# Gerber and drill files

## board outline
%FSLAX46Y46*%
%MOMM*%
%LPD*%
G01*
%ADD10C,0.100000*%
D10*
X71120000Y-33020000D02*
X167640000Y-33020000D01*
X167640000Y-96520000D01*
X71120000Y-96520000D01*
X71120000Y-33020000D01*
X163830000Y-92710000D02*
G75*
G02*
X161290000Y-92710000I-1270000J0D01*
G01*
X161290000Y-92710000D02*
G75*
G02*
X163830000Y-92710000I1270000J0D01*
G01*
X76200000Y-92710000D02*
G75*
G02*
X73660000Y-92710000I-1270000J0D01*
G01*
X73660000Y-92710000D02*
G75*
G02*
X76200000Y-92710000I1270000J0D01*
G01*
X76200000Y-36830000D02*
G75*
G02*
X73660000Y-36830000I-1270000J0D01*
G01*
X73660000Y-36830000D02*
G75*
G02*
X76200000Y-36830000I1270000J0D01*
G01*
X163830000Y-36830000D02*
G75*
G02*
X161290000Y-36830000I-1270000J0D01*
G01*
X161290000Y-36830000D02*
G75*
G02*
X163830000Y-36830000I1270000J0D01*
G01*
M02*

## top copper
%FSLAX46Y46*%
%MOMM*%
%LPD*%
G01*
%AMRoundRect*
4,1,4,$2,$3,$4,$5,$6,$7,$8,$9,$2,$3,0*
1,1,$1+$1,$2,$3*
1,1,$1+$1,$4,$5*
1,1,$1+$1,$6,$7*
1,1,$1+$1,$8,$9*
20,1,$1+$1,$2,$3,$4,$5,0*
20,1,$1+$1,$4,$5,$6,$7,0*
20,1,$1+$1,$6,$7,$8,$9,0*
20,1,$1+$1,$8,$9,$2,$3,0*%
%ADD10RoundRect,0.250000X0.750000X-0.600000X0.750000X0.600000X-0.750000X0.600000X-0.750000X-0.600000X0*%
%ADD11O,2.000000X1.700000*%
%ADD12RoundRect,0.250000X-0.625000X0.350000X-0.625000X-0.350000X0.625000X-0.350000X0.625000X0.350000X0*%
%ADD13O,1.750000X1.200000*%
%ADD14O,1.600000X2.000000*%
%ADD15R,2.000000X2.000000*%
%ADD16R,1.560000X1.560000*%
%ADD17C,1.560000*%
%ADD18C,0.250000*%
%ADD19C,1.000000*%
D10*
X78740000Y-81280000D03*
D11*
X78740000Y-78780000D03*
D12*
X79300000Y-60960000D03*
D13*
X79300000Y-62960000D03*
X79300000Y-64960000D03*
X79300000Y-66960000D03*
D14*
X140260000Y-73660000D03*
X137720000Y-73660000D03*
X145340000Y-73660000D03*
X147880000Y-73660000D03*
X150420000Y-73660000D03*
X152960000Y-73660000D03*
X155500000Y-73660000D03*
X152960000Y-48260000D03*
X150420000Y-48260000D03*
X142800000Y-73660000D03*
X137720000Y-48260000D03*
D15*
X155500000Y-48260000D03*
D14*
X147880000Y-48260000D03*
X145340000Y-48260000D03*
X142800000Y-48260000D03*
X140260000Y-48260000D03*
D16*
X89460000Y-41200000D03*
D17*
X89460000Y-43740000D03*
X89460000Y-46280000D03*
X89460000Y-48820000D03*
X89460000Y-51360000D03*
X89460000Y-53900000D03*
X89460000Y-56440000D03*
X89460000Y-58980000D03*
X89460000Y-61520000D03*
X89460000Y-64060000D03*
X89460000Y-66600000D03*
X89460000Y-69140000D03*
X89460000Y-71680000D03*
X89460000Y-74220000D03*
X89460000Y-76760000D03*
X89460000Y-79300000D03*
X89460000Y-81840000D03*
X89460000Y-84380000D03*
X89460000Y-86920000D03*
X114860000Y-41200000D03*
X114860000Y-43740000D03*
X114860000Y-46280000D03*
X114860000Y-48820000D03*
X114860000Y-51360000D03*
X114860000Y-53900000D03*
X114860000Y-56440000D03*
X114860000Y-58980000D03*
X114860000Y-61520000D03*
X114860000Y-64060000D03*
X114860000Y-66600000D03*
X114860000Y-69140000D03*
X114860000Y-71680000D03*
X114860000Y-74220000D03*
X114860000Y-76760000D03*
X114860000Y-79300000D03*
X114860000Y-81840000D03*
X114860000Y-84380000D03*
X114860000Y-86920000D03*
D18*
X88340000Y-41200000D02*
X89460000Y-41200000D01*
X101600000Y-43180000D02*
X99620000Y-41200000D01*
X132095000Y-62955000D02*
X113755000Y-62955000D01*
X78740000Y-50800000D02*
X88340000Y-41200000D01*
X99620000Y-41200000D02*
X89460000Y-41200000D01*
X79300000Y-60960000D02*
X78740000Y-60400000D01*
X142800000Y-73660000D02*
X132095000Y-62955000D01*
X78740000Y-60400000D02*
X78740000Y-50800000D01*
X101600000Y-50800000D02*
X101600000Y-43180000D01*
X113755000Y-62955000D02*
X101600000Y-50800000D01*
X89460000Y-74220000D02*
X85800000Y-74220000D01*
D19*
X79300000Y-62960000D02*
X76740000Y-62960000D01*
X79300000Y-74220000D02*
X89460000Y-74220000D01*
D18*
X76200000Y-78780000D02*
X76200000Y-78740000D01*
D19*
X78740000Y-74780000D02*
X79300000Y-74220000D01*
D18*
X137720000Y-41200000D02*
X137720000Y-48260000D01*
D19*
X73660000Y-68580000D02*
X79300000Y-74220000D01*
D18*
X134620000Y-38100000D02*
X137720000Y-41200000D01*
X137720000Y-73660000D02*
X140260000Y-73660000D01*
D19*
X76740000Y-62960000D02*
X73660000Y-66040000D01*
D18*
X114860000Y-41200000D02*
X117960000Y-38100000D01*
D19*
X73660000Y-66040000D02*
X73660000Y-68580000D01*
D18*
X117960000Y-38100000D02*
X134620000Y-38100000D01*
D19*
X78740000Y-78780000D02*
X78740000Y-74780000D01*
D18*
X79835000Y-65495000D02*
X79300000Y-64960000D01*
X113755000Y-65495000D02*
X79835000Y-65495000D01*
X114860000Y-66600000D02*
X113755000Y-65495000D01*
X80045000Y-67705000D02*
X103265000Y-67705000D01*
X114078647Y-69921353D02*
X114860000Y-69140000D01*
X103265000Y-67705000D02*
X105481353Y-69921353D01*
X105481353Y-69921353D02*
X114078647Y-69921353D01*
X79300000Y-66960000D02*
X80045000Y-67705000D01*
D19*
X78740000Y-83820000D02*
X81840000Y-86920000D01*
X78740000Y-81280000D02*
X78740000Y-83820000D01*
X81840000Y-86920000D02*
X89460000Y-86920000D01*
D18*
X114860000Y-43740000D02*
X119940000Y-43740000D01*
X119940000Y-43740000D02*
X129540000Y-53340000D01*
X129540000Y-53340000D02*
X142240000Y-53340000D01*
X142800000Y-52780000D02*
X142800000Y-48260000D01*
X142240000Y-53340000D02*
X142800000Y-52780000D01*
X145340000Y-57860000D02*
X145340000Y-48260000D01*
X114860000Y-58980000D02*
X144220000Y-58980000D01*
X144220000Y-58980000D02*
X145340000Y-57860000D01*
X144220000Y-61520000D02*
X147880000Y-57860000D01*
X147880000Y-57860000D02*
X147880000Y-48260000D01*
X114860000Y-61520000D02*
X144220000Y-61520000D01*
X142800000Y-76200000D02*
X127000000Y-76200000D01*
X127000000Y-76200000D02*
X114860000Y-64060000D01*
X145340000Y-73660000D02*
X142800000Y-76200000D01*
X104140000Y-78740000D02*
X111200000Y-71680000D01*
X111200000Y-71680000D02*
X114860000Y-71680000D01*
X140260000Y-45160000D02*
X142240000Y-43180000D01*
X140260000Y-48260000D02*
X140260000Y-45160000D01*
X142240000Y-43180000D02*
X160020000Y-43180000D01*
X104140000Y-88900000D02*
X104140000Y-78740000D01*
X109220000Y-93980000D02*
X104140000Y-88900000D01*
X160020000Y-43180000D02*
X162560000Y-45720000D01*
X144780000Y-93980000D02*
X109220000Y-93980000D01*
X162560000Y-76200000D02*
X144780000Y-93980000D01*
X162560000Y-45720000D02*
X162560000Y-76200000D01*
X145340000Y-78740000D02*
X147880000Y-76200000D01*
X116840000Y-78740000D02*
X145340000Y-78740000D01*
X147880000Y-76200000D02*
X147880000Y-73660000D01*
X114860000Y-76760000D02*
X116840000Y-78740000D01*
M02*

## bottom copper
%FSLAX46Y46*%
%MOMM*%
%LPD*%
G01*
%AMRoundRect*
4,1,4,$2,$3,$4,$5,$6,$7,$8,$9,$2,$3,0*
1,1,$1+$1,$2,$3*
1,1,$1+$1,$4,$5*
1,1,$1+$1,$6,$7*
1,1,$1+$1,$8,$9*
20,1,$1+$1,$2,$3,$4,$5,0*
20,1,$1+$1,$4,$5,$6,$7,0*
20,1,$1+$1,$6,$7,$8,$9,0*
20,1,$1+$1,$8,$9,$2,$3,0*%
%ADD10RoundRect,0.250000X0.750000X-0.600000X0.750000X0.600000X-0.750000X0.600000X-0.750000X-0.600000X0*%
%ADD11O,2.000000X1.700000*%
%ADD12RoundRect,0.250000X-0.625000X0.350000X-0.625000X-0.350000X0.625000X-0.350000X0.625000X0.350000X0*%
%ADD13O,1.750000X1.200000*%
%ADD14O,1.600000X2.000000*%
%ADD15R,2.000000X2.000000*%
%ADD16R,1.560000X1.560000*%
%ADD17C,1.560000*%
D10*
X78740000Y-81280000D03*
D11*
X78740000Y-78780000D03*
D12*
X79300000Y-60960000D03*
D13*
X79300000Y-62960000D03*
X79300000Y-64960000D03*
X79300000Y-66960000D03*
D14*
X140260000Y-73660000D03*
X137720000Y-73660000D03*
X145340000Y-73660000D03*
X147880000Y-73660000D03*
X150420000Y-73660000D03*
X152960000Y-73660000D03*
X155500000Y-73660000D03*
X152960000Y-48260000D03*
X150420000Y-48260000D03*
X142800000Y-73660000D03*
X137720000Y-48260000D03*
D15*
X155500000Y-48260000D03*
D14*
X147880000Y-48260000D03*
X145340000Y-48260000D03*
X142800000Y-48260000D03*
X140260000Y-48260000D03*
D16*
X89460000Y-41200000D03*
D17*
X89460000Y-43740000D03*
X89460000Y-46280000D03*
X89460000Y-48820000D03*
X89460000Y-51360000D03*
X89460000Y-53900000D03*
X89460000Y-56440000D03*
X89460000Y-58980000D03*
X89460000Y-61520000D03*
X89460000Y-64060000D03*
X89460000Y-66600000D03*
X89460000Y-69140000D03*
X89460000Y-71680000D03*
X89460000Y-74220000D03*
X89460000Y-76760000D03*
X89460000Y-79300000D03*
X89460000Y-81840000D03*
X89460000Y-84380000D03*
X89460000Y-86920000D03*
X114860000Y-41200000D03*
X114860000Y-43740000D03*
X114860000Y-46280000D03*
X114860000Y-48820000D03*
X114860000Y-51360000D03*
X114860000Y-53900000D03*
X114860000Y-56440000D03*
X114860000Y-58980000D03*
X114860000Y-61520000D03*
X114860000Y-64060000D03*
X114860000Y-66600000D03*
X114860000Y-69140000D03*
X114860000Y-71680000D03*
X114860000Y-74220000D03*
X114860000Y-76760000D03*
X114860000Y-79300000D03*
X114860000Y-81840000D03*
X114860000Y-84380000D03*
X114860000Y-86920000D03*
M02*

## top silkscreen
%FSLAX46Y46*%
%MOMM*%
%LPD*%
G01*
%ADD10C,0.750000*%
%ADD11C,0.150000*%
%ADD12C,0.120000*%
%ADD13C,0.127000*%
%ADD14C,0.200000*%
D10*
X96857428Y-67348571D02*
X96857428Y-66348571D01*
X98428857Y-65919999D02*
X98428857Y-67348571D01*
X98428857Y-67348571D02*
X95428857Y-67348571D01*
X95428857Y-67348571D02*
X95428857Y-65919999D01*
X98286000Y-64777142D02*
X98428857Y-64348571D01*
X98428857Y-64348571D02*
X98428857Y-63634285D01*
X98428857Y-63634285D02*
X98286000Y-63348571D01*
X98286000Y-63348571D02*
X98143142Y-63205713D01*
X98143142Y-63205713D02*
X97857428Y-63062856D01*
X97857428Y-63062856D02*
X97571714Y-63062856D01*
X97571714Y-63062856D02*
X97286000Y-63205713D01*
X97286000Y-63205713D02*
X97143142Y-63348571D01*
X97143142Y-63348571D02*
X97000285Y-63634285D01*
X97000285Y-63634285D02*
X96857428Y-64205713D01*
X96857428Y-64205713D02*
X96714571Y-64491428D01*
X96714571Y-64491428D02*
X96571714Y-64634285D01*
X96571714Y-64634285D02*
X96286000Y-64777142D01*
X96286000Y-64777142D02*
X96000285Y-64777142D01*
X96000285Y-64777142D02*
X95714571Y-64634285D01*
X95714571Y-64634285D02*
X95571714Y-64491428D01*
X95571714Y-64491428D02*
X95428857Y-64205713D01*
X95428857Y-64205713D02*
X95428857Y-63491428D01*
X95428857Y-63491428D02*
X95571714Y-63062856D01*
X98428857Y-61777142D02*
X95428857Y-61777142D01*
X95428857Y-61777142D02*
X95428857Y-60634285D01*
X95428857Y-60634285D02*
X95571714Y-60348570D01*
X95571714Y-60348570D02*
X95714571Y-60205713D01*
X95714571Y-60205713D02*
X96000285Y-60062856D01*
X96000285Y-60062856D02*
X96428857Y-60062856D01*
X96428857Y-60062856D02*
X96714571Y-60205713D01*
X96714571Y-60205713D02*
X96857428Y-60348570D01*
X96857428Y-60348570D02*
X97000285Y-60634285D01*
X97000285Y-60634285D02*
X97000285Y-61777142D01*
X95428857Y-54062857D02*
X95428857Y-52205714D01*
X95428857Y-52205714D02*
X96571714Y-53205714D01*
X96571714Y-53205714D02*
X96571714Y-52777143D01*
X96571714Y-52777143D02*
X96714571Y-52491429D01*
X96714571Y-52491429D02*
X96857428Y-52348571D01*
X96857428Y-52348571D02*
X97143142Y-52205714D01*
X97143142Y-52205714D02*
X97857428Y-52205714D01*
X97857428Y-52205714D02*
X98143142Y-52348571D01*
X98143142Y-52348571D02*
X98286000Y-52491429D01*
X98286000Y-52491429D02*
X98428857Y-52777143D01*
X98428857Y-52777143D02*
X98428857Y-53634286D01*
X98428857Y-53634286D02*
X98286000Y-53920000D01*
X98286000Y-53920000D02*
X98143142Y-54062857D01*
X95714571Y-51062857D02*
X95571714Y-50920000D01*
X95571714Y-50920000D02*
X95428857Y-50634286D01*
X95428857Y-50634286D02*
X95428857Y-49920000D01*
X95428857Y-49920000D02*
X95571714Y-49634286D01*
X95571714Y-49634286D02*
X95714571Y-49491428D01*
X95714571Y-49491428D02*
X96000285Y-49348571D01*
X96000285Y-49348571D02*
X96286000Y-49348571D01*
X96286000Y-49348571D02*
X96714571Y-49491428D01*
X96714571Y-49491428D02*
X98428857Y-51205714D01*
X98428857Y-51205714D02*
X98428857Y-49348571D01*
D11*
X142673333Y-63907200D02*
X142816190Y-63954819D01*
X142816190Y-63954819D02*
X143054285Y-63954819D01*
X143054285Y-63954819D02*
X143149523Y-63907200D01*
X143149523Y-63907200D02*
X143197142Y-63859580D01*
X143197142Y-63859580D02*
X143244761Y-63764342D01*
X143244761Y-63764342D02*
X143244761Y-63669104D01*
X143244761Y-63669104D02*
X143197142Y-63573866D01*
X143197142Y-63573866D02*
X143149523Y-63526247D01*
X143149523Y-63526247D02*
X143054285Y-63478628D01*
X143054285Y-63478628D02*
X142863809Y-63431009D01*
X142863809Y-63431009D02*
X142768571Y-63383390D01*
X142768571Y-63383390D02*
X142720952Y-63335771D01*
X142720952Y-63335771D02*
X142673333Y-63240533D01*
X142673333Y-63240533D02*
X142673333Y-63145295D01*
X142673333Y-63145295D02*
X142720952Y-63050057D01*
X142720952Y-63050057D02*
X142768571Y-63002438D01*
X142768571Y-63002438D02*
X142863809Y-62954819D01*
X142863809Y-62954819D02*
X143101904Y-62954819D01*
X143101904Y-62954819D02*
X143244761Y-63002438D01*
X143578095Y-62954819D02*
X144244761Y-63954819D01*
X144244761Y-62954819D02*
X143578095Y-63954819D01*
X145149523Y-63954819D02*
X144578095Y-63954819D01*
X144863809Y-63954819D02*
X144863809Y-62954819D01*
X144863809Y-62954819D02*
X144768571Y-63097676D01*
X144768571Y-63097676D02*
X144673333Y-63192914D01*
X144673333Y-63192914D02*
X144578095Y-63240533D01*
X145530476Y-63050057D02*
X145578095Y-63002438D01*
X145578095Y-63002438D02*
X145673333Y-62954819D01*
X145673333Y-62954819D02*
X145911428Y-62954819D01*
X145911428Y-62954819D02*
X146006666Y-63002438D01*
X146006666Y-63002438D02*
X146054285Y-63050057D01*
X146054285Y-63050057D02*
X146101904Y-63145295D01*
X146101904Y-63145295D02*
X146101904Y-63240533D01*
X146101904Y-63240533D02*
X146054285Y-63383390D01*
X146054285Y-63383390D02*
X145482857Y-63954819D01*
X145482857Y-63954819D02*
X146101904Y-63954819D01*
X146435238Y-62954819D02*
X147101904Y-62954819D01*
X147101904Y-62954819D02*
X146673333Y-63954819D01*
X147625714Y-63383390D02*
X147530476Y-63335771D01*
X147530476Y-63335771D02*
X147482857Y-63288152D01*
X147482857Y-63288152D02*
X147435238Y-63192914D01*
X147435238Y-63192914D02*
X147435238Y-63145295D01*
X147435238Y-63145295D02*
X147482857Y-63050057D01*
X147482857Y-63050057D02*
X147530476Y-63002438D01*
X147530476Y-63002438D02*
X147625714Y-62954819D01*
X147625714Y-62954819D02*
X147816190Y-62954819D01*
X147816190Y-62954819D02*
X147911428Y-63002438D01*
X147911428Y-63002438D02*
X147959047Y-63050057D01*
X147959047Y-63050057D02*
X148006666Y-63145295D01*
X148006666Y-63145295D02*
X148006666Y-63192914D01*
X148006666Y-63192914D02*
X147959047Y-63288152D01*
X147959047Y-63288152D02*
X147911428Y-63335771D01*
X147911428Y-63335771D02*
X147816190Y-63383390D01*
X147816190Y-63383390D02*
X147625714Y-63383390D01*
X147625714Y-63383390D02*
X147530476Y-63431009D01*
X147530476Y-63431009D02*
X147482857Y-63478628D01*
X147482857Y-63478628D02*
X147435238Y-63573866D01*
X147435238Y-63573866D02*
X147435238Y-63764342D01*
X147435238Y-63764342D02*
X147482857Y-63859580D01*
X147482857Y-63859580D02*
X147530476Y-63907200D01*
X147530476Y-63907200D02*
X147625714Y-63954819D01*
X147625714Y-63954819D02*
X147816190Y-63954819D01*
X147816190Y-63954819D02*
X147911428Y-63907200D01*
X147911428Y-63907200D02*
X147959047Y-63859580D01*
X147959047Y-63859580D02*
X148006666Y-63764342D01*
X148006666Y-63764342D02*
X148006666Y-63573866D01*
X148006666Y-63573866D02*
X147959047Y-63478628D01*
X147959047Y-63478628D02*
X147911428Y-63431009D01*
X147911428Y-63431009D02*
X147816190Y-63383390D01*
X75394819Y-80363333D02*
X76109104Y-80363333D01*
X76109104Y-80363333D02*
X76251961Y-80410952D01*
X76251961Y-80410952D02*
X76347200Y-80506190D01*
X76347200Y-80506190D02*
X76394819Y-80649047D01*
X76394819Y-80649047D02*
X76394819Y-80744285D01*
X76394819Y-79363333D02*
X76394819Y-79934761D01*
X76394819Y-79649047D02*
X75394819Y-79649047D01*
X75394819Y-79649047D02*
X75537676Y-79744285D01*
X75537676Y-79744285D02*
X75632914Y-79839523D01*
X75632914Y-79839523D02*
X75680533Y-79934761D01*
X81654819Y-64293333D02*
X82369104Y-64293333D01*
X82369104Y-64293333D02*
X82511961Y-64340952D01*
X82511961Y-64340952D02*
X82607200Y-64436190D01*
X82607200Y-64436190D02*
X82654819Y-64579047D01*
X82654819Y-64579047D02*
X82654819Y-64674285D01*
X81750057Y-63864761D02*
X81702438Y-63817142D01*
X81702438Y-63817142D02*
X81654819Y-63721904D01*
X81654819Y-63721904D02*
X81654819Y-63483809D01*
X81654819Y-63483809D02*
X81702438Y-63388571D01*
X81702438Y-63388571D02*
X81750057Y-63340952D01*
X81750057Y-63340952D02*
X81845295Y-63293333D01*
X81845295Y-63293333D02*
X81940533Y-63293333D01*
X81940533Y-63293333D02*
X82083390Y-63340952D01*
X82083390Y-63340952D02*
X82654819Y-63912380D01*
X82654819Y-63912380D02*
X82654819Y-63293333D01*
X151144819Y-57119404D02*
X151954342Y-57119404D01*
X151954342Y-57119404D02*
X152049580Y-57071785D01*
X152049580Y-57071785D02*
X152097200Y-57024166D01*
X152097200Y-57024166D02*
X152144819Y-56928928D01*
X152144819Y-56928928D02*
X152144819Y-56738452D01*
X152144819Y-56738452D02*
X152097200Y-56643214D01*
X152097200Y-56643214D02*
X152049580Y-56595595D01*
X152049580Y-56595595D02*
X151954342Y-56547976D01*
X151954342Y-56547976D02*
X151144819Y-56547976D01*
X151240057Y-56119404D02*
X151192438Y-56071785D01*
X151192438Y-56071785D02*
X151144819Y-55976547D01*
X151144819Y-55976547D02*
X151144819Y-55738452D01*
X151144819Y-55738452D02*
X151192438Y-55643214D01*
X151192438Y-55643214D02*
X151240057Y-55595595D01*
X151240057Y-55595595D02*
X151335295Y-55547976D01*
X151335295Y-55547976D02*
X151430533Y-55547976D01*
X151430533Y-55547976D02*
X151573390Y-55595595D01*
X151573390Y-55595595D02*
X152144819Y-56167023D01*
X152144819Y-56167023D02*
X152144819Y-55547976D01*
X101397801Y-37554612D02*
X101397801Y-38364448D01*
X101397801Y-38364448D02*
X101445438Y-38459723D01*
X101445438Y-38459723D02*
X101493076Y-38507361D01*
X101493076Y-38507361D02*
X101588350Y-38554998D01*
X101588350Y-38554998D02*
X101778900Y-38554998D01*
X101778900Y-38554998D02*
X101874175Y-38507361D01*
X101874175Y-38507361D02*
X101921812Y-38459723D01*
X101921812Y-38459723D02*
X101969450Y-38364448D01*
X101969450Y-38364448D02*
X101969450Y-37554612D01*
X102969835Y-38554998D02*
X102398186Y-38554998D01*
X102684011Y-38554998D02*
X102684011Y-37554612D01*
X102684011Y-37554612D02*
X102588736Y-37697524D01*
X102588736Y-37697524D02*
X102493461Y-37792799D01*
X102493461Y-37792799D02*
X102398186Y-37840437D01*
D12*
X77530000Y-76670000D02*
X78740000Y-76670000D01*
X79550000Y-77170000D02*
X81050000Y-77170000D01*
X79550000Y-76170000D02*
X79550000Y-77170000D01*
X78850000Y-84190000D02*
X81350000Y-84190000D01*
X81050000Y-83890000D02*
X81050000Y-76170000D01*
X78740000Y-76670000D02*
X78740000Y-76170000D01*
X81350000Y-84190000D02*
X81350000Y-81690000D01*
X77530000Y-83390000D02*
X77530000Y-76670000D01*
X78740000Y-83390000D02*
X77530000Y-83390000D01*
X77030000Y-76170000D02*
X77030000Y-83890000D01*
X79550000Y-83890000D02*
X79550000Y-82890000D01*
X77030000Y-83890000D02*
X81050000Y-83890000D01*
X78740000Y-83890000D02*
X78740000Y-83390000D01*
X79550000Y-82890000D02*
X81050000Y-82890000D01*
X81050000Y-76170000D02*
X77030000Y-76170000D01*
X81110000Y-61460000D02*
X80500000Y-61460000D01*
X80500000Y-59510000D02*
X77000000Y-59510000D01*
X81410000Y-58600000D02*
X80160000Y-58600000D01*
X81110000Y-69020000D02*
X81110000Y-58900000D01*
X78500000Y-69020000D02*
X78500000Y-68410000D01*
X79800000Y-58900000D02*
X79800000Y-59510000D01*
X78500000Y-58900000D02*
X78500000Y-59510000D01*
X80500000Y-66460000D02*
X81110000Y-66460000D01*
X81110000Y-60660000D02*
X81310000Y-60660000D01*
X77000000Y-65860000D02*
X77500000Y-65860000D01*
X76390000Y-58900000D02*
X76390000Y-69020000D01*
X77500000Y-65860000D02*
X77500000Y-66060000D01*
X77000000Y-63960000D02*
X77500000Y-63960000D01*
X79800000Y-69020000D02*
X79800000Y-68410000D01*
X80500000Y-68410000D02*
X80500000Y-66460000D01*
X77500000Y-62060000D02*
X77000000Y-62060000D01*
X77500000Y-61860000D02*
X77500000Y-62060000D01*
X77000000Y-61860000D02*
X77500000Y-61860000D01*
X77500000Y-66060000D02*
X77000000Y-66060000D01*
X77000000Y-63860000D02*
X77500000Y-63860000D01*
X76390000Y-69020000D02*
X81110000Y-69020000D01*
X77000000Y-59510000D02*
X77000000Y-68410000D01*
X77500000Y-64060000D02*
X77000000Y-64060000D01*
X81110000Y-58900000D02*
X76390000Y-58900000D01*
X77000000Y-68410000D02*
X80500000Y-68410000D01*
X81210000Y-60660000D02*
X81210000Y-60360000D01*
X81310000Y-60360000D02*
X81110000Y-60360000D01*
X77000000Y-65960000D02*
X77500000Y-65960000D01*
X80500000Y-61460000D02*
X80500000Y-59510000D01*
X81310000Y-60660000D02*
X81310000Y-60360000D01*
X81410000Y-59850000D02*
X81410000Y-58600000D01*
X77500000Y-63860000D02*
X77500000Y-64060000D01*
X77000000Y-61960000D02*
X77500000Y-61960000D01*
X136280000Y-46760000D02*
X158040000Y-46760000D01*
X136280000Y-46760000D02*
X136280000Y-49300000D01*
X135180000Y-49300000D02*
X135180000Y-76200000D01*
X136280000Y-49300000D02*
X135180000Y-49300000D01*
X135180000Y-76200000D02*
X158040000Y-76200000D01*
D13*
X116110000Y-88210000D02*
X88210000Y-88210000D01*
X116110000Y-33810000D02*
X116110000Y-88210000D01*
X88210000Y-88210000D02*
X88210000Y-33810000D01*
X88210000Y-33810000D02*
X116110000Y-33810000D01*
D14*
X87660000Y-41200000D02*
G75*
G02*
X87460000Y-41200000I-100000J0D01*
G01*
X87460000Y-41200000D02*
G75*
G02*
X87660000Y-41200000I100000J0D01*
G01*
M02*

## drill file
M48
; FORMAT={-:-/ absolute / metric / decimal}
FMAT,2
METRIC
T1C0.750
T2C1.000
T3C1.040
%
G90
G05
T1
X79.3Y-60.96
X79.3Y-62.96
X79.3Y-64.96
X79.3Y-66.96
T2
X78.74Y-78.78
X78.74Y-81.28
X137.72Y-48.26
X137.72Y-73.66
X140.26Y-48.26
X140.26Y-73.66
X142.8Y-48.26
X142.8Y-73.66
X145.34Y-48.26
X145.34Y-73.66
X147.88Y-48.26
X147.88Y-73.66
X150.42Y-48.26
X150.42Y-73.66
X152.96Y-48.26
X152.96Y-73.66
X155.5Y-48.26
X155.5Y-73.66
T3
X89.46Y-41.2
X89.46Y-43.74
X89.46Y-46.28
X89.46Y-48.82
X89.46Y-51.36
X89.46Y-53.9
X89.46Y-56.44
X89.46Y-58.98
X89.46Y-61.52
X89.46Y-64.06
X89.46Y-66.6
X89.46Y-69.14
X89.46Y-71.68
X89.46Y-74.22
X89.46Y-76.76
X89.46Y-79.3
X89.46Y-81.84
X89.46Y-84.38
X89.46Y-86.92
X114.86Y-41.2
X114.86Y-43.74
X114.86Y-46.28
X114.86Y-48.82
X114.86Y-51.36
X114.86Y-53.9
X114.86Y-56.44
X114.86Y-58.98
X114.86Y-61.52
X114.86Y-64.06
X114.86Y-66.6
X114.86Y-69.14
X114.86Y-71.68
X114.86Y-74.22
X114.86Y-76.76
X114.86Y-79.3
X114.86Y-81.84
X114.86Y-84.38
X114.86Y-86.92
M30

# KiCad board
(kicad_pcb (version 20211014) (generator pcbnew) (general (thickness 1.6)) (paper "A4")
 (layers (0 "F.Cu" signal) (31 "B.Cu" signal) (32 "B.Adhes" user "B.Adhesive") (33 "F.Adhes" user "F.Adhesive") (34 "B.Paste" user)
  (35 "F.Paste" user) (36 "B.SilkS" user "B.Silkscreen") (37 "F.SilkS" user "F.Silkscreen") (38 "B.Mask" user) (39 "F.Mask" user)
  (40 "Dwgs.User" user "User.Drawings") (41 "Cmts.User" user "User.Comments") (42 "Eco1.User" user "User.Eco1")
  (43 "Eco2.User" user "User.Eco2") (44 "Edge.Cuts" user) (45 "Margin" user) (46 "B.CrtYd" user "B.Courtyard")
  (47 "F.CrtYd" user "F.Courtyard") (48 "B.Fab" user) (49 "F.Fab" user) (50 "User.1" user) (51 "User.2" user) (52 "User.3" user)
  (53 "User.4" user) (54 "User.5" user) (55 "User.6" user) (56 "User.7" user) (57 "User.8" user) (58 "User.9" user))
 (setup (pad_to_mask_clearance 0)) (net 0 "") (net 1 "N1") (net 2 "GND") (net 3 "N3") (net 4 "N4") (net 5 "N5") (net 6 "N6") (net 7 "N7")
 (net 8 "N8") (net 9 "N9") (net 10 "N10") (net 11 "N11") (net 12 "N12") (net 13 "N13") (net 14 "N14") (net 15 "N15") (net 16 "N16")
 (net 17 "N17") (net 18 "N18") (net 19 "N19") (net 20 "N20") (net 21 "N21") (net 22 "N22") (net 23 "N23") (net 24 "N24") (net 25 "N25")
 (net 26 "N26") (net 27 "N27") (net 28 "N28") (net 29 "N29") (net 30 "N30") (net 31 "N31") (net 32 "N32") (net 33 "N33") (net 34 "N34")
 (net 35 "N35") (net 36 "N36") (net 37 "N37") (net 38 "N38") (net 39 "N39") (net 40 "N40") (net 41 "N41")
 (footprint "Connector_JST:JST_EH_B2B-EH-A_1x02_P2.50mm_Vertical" (layer "F.Cu") (at 78.74 81.28 90)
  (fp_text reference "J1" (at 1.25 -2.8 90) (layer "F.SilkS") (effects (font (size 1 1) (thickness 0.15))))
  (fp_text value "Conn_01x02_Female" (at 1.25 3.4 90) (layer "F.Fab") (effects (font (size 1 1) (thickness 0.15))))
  (fp_line (start 4.61 -1.21) (end 4.61 0) (layer "F.SilkS") (width 0.12))
  (fp_line (start 4.11 0.81) (end 4.11 2.31) (layer "F.SilkS") (width 0.12))
  (fp_line (start 5.11 0.81) (end 4.11 0.81) (layer "F.SilkS") (width 0.12))
  (fp_line (start -2.91 0.11) (end -2.91 2.61) (layer "F.SilkS") (width 0.12))
  (fp_line (start -2.61 2.31) (end 5.11 2.31) (layer "F.SilkS") (width 0.12))
  (fp_line (start 4.61 0) (end 5.11 0) (layer "F.SilkS") (width 0.12))
  (fp_line (start -2.91 2.61) (end -0.41 2.61) (layer "F.SilkS") (width 0.12))
  (fp_line (start -2.11 -1.21) (end 4.61 -1.21) (layer "F.SilkS") (width 0.12))
  (fp_line (start -2.11 0) (end -2.11 -1.21) (layer "F.SilkS") (width 0.12))
  (fp_line (start 5.11 -1.71) (end -2.61 -1.71) (layer "F.SilkS") (width 0.12))
  (fp_line (start -2.61 0.81) (end -1.61 0.81) (layer "F.SilkS") (width 0.12))
  (fp_line (start -2.61 -1.71) (end -2.61 2.31) (layer "F.SilkS") (width 0.12))
  (fp_line (start -2.61 0) (end -2.11 0) (layer "F.SilkS") (width 0.12))
  (fp_line (start -1.61 0.81) (end -1.61 2.31) (layer "F.SilkS") (width 0.12))
  (fp_line (start 5.11 2.31) (end 5.11 -1.71) (layer "F.SilkS") (width 0.12))
  (pad "1" thru_hole roundrect (at 0 0 90) (size 1.7 2) (drill 1) (layers *.Cu *.Mask) (roundrect_rratio 0.147059) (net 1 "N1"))
  (pad "2" thru_hole oval (at 2.5 0 90) (size 1.7 2) (drill 1) (layers *.Cu *.Mask) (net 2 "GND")))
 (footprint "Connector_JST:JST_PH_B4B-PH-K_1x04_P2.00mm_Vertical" (layer "F.Cu") (at 79.3 60.96 -90)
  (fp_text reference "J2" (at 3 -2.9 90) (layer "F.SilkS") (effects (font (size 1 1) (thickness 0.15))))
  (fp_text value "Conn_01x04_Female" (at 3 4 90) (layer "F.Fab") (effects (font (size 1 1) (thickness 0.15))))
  (fp_line (start 0.5 -1.81) (end 0.5 -1.2) (layer "F.SilkS") (width 0.12))
  (fp_line (start -1.45 -1.2) (end -1.45 2.3) (layer "F.SilkS") (width 0.12))
  (fp_line (start -2.36 -2.11) (end -2.36 -0.86) (layer "F.SilkS") (width 0.12))
  (fp_line (start 8.06 -1.81) (end -2.06 -1.81) (layer "F.SilkS") (width 0.12))
  (fp_line (start 8.06 0.8) (end 7.45 0.8) (layer "F.SilkS") (width 0.12))
  (fp_line (start -2.06 -0.5) (end -1.45 -0.5) (layer "F.SilkS") (width 0.12))
  (fp_line (start -2.06 0.8) (end -1.45 0.8) (layer "F.SilkS") (width 0.12))
  (fp_line (start 5.5 -1.2) (end 5.5 -1.81) (layer "F.SilkS") (width 0.12))
  (fp_line (start -0.3 -1.81) (end -0.3 -2.01) (layer "F.SilkS") (width 0.12))
  (fp_line (start 4.9 2.3) (end 4.9 1.8) (layer "F.SilkS") (width 0.12))
  (fp_line (start -2.06 2.91) (end 8.06 2.91) (layer "F.SilkS") (width 0.12))
  (fp_line (start 4.9 1.8) (end 5.1 1.8) (layer "F.SilkS") (width 0.12))
  (fp_line (start 3 2.3) (end 3 1.8) (layer "F.SilkS") (width 0.12))
  (fp_line (start 8.06 -0.5) (end 7.45 -0.5) (layer "F.SilkS") (width 0.12))
  (fp_line (start 7.45 -1.2) (end 5.5 -1.2) (layer "F.SilkS") (width 0.12))
  (fp_line (start 1.1 1.8) (end 1.1 2.3) (layer "F.SilkS") (width 0.12))
  (fp_line (start 0.9 1.8) (end 1.1 1.8) (layer "F.SilkS") (width 0.12))
  (fp_line (start 0.9 2.3) (end 0.9 1.8) (layer "F.SilkS") (width 0.12))
  (fp_line (start 5.1 1.8) (end 5.1 2.3) (layer "F.SilkS") (width 0.12))
  (fp_line (start 2.9 2.3) (end 2.9 1.8) (layer "F.SilkS") (width 0.12))
  (fp_line (start 8.06 2.91) (end 8.06 -1.81) (layer "F.SilkS") (width 0.12))
  (fp_line (start -1.45 2.3) (end 7.45 2.3) (layer "F.SilkS") (width 0.12))
  (fp_line (start 3.1 1.8) (end 3.1 2.3) (layer "F.SilkS") (width 0.12))
  (fp_line (start -2.06 -1.81) (end -2.06 2.91) (layer "F.SilkS") (width 0.12))
  (fp_line (start 7.45 2.3) (end 7.45 -1.2) (layer "F.SilkS") (width 0.12))
  (fp_line (start -0.3 -1.91) (end -0.6 -1.91) (layer "F.SilkS") (width 0.12))
  (fp_line (start -0.6 -2.01) (end -0.6 -1.81) (layer "F.SilkS") (width 0.12))
  (fp_line (start 5 2.3) (end 5 1.8) (layer "F.SilkS") (width 0.12))
  (fp_line (start 0.5 -1.2) (end -1.45 -1.2) (layer "F.SilkS") (width 0.12))
  (fp_line (start -0.3 -2.01) (end -0.6 -2.01) (layer "F.SilkS") (width 0.12))
  (fp_line (start -1.11 -2.11) (end -2.36 -2.11) (layer "F.SilkS") (width 0.12))
  (fp_line (start 2.9 1.8) (end 3.1 1.8) (layer "F.SilkS") (width 0.12))
  (fp_line (start 1 2.3) (end 1 1.8) (layer "F.SilkS") (width 0.12))
  (pad "1" thru_hole roundrect (at 0 0 270) (size 1.2 1.75) (drill 0.75) (layers *.Cu *.Mask) (roundrect_rratio 0.208333) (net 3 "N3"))
  (pad "2" thru_hole oval (at 2 0 270) (size 1.2 1.75) (drill 0.75) (layers *.Cu *.Mask) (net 2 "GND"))
  (pad "3" thru_hole oval (at 4 0 270) (size 1.2 1.75) (drill 0.75) (layers *.Cu *.Mask) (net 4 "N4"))
  (pad "4" thru_hole oval (at 6 0 270) (size 1.2 1.75) (drill 0.75) (layers *.Cu *.Mask) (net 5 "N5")))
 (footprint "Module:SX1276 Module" (layer "F.Cu") (at 155.5 48.26 -90)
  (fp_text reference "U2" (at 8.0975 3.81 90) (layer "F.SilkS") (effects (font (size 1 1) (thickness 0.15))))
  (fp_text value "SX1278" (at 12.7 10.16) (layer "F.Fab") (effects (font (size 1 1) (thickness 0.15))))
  (fp_line (start -1.5 19.22) (end -1.5 -2.54) (layer "F.SilkS") (width 0.12))
  (fp_line (start -1.5 19.22) (end 1.04 19.22) (layer "F.SilkS") (width 0.12))
  (fp_line (start 1.04 20.32) (end 27.94 20.32) (layer "F.SilkS") (width 0.12))
  (fp_line (start 1.04 19.22) (end 1.04 20.32) (layer "F.SilkS") (width 0.12))
  (fp_line (start 27.94 20.32) (end 27.94 -2.54) (layer "F.SilkS") (width 0.12))
  (pad "2" thru_hole oval (at 25.4 15.24 270) (size 2 1.6) (drill 1) (layers *.Cu *.Mask) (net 2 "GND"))
  (pad "4" thru_hole oval (at 25.4 17.78 270) (size 2 1.6) (drill 1) (layers *.Cu *.Mask) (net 2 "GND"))
  (pad "7" thru_hole oval (at 25.4 10.16 270) (size 2 1.6) (drill 1) (layers *.Cu *.Mask) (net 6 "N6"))
  (pad "8" thru_hole oval (at 25.4 7.62 270) (size 2 1.6) (drill 1) (layers *.Cu *.Mask) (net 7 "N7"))
  (pad "9" thru_hole oval (at 25.4 5.08 270) (size 2 1.6) (drill 1) (layers *.Cu *.Mask) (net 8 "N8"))
  (pad "10" thru_hole oval (at 25.4 2.54 270) (size 2 1.6) (drill 1) (layers *.Cu *.Mask) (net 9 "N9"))
  (pad "11" thru_hole oval (at 25.4 0 270) (size 2 1.6) (drill 1) (layers *.Cu *.Mask) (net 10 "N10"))
  (pad "12" thru_hole oval (at 0 2.54 270) (size 2 1.6) (drill 1) (layers *.Cu *.Mask) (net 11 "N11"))
  (pad "13" thru_hole oval (at 0 5.08 270) (size 2 1.6) (drill 1) (layers *.Cu *.Mask) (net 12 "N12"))
  (pad "14" thru_hole oval (at 25.4 12.7 270) (size 2 1.6) (drill 1) (layers *.Cu *.Mask) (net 3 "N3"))
  (pad "15" thru_hole oval (at 0 17.78 270) (size 2 1.6) (drill 1) (layers *.Cu *.Mask) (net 2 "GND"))
  (pad "15" thru_hole rect (at 0 0 270) (size 2 2) (drill 1) (layers *.Cu *.Mask) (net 2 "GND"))
  (pad "16" thru_hole oval (at 0 7.62 270) (size 2 1.6) (drill 1) (layers *.Cu *.Mask) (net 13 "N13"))
  (pad "17" thru_hole oval (at 0 10.16 270) (size 2 1.6) (drill 1) (layers *.Cu *.Mask) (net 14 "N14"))
  (pad "18" thru_hole oval (at 0 12.7 270) (size 2 1.6) (drill 1) (layers *.Cu *.Mask) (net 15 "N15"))
  (pad "19" thru_hole oval (at 0 15.24 270) (size 2 1.6) (drill 1) (layers *.Cu *.Mask) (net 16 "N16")))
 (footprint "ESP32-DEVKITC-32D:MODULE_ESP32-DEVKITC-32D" (layer "F.Cu") (at 102.16 60.96)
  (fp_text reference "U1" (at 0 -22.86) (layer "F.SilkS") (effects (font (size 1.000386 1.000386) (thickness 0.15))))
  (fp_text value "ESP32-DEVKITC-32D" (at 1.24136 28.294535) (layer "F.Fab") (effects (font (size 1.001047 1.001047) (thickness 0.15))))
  (fp_line (start 13.95 27.25) (end -13.95 27.25) (layer "F.SilkS") (width 0.127))
  (fp_line (start 13.95 -27.15) (end 13.95 27.25) (layer "F.SilkS") (width 0.127))
  (fp_line (start -13.95 27.25) (end -13.95 -27.15) (layer "F.SilkS") (width 0.127))
  (fp_line (start -13.95 -27.15) (end 13.95 -27.15) (layer "F.SilkS") (width 0.127))
  (fp_circle (center -14.6 -19.76) (end -14.5 -19.76) (layer "F.SilkS") (width 0.2) (fill none))
  (pad "J2-1" thru_hole rect locked (at -12.7 -19.76) (size 1.56 1.56) (drill 1.04) (layers *.Cu *.Mask) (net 3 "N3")
   (solder_mask_margin 0.102))
  (pad "J2-2" thru_hole circle locked (at -12.7 -17.22) (size 1.56 1.56) (drill 1.04) (layers *.Cu *.Mask) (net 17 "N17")
   (solder_mask_margin 0.102))
  (pad "J2-3" thru_hole circle locked (at -12.7 -14.68) (size 1.56 1.56) (drill 1.04) (layers *.Cu *.Mask) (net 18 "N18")
   (solder_mask_margin 0.102))
  (pad "J2-4" thru_hole circle locked (at -12.7 -12.14) (size 1.56 1.56) (drill 1.04) (layers *.Cu *.Mask) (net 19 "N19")
   (solder_mask_margin 0.102))
  (pad "J2-5" thru_hole circle locked (at -12.7 -9.6) (size 1.56 1.56) (drill 1.04) (layers *.Cu *.Mask) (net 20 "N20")
   (solder_mask_margin 0.102))
  (pad "J2-6" thru_hole circle locked (at -12.7 -7.06) (size 1.56 1.56) (drill 1.04) (layers *.Cu *.Mask) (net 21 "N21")
   (solder_mask_margin 0.102))
  (pad "J2-7" thru_hole circle locked (at -12.7 -4.52) (size 1.56 1.56) (drill 1.04) (layers *.Cu *.Mask) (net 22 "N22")
   (solder_mask_margin 0.102))
  (pad "J2-8" thru_hole circle locked (at -12.7 -1.98) (size 1.56 1.56) (drill 1.04) (layers *.Cu *.Mask) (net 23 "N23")
   (solder_mask_margin 0.102))
  (pad "J2-9" thru_hole circle locked (at -12.7 0.56) (size 1.56 1.56) (drill 1.04) (layers *.Cu *.Mask) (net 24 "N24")
   (solder_mask_margin 0.102))
  (pad "J2-10" thru_hole circle locked (at -12.7 3.1) (size 1.56 1.56) (drill 1.04) (layers *.Cu *.Mask) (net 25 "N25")
   (solder_mask_margin 0.102))
  (pad "J2-11" thru_hole circle locked (at -12.7 5.64) (size 1.56 1.56) (drill 1.04) (layers *.Cu *.Mask) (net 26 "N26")
   (solder_mask_margin 0.102))
  (pad "J2-12" thru_hole circle locked (at -12.7 8.18) (size 1.56 1.56) (drill 1.04) (layers *.Cu *.Mask) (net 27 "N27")
   (solder_mask_margin 0.102))
  (pad "J2-13" thru_hole circle locked (at -12.7 10.72) (size 1.56 1.56) (drill 1.04) (layers *.Cu *.Mask) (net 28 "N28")
   (solder_mask_margin 0.102))
  (pad "J2-14" thru_hole circle locked (at -12.7 13.26) (size 1.56 1.56) (drill 1.04) (layers *.Cu *.Mask) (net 2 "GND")
   (solder_mask_margin 0.102))
  (pad "J2-15" thru_hole circle locked (at -12.7 15.8) (size 1.56 1.56) (drill 1.04) (layers *.Cu *.Mask) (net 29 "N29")
   (solder_mask_margin 0.102))
  (pad "J2-16" thru_hole circle locked (at -12.7 18.34) (size 1.56 1.56) (drill 1.04) (layers *.Cu *.Mask) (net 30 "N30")
   (solder_mask_margin 0.102))
  (pad "J2-17" thru_hole circle locked (at -12.7 20.88) (size 1.56 1.56) (drill 1.04) (layers *.Cu *.Mask) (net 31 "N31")
   (solder_mask_margin 0.102))
  (pad "J2-18" thru_hole circle locked (at -12.7 23.42) (size 1.56 1.56) (drill 1.04) (layers *.Cu *.Mask) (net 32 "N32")
   (solder_mask_margin 0.102))
  (pad "J2-19" thru_hole circle locked (at -12.7 25.96) (size 1.56 1.56) (drill 1.04) (layers *.Cu *.Mask) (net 1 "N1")
   (solder_mask_margin 0.102))
  (pad "J3-1" thru_hole circle locked (at 12.7 -19.76) (size 1.56 1.56) (drill 1.04) (layers *.Cu *.Mask) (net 2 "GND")
   (solder_mask_margin 0.102))
  (pad "J3-2" thru_hole circle locked (at 12.7 -17.22) (size 1.56 1.56) (drill 1.04) (layers *.Cu *.Mask) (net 15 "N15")
   (solder_mask_margin 0.102))
  (pad "J3-3" thru_hole circle locked (at 12.7 -14.68) (size 1.56 1.56) (drill 1.04) (layers *.Cu *.Mask) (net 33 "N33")
   (solder_mask_margin 0.102))
  (pad "J3-4" thru_hole circle locked (at 12.7 -12.14) (size 1.56 1.56) (drill 1.04) (layers *.Cu *.Mask) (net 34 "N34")
   (solder_mask_margin 0.102))
  (pad "J3-5" thru_hole circle locked (at 12.7 -9.6) (size 1.56 1.56) (drill 1.04) (layers *.Cu *.Mask) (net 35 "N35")
   (solder_mask_margin 0.102))
  (pad "J3-6" thru_hole circle locked (at 12.7 -7.06) (size 1.56 1.56) (drill 1.04) (layers *.Cu *.Mask) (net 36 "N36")
   (solder_mask_margin 0.102))
  (pad "J3-7" thru_hole circle locked (at 12.7 -4.52) (size 1.56 1.56) (drill 1.04) (layers *.Cu *.Mask) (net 2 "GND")
   (solder_mask_margin 0.102))
  (pad "J3-8" thru_hole circle locked (at 12.7 -1.98) (size 1.56 1.56) (drill 1.04) (layers *.Cu *.Mask) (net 14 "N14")
   (solder_mask_margin 0.102))
  (pad "J3-9" thru_hole circle locked (at 12.7 0.56) (size 1.56 1.56) (drill 1.04) (layers *.Cu *.Mask) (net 13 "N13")
   (solder_mask_margin 0.102))
  (pad "J3-10" thru_hole circle locked (at 12.7 3.1) (size 1.56 1.56) (drill 1.04) (layers *.Cu *.Mask) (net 6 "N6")
   (solder_mask_margin 0.102))
  (pad "J3-11" thru_hole circle locked (at 12.7 5.64) (size 1.56 1.56) (drill 1.04) (layers *.Cu *.Mask) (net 4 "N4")
   (solder_mask_margin 0.102))
  (pad "J3-12" thru_hole circle locked (at 12.7 8.18) (size 1.56 1.56) (drill 1.04) (layers *.Cu *.Mask) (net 5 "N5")
   (solder_mask_margin 0.102))
  (pad "J3-13" thru_hole circle locked (at 12.7 10.72) (size 1.56 1.56) (drill 1.04) (layers *.Cu *.Mask) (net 16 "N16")
   (solder_mask_margin 0.102))
  (pad "J3-14" thru_hole circle locked (at 12.7 13.26) (size 1.56 1.56) (drill 1.04) (layers *.Cu *.Mask) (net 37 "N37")
   (solder_mask_margin 0.102))
  (pad "J3-15" thru_hole circle locked (at 12.7 15.8) (size 1.56 1.56) (drill 1.04) (layers *.Cu *.Mask) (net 7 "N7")
   (solder_mask_margin 0.102))
  (pad "J3-16" thru_hole circle locked (at 12.7 18.34) (size 1.56 1.56) (drill 1.04) (layers *.Cu *.Mask) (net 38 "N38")
   (solder_mask_margin 0.102))
  (pad "J3-17" thru_hole circle locked (at 12.7 20.88) (size 1.56 1.56) (drill 1.04) (layers *.Cu *.Mask) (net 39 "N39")
   (solder_mask_margin 0.102))
  (pad "J3-18" thru_hole circle locked (at 12.7 23.42) (size 1.56 1.56) (drill 1.04) (layers *.Cu *.Mask) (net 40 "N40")
   (solder_mask_margin 0.102))
  (pad "J3-19" thru_hole circle locked (at 12.7 25.96) (size 1.56 1.56) (drill 1.04) (layers *.Cu *.Mask) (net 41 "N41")
   (solder_mask_margin 0.102)))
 (gr_rect (start 71.12 33.02) (end 167.64 96.52) (layer "Edge.Cuts") (width 0.1) (fill none))
 (gr_circle (center 162.56 92.71) (end 162.56 93.98) (layer "Edge.Cuts") (width 0.1) (fill none))
 (gr_circle (center 74.93 92.71) (end 74.93 93.98) (layer "Edge.Cuts") (width 0.1) (fill none))
 (gr_circle (center 74.93 36.83) (end 74.93 38.1) (layer "Edge.Cuts") (width 0.1) (fill none))
 (gr_circle (center 162.56 36.83) (end 162.56 38.1) (layer "Edge.Cuts") (width 0.1) (fill none))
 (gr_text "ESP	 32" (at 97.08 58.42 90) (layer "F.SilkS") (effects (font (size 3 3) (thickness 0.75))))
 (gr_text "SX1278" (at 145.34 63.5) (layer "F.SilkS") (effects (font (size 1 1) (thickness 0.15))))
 (segment (start 88.34 41.2) (end 89.46 41.2) (width 0.25) (layer "F.Cu") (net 3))
 (segment (start 101.6 43.18) (end 99.62 41.2) (width 0.25) (layer "F.Cu") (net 3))
 (segment (start 132.095 62.955) (end 113.755 62.955) (width 0.25) (layer "F.Cu") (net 3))
 (segment (start 78.74 50.8) (end 88.34 41.2) (width 0.25) (layer "F.Cu") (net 3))
 (segment (start 99.62 41.2) (end 89.46 41.2) (width 0.25) (layer "F.Cu") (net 3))
 (segment (start 79.3 60.96) (end 78.74 60.4) (width 0.25) (layer "F.Cu") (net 3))
 (segment (start 142.8 73.66) (end 132.095 62.955) (width 0.25) (layer "F.Cu") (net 3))
 (segment (start 78.74 60.4) (end 78.74 50.8) (width 0.25) (layer "F.Cu") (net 3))
 (segment (start 101.6 50.8) (end 101.6 43.18) (width 0.25) (layer "F.Cu") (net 3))
 (segment (start 113.755 62.955) (end 101.6 50.8) (width 0.25) (layer "F.Cu") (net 3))
 (segment (start 89.46 74.22) (end 85.8 74.22) (width 0.25) (layer "F.Cu") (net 2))
 (segment (start 79.3 62.96) (end 76.74 62.96) (width 1) (layer "F.Cu") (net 2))
 (segment (start 79.3 74.22) (end 89.46 74.22) (width 1) (layer "F.Cu") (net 2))
 (segment (start 76.2 78.78) (end 76.2 78.74) (width 0.25) (layer "F.Cu") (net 2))
 (segment (start 78.74 74.78) (end 79.3 74.22) (width 1) (layer "F.Cu") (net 2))
 (segment (start 137.72 41.2) (end 137.72 48.26) (width 0.25) (layer "F.Cu") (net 2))
 (segment (start 73.66 68.58) (end 79.3 74.22) (width 1) (layer "F.Cu") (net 2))
 (segment (start 134.62 38.1) (end 137.72 41.2) (width 0.25) (layer "F.Cu") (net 2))
 (segment (start 137.72 73.66) (end 140.26 73.66) (width 0.25) (layer "F.Cu") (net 2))
 (segment (start 76.74 62.96) (end 73.66 66.04) (width 1) (layer "F.Cu") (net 2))
 (segment (start 114.86 41.2) (end 117.96 38.1) (width 0.25) (layer "F.Cu") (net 2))
 (segment (start 73.66 66.04) (end 73.66 68.58) (width 1) (layer "F.Cu") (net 2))
 (segment (start 117.96 38.1) (end 134.62 38.1) (width 0.25) (layer "F.Cu") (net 2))
 (segment (start 78.74 78.78) (end 78.74 74.78) (width 1) (layer "F.Cu") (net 2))
 (segment (start 79.835 65.495) (end 79.3 64.96) (width 0.25) (layer "F.Cu") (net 4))
 (segment (start 113.755 65.495) (end 79.835 65.495) (width 0.25) (layer "F.Cu") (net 4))
 (segment (start 114.86 66.6) (end 113.755 65.495) (width 0.25) (layer "F.Cu") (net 4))
 (segment (start 80.045 67.705) (end 103.265 67.705) (width 0.25) (layer "F.Cu") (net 5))
 (segment (start 114.078647 69.921353) (end 114.86 69.14) (width 0.25) (layer "F.Cu") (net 5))
 (segment (start 103.265 67.705) (end 105.481353 69.921353) (width 0.25) (layer "F.Cu") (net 5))
 (segment (start 105.481353 69.921353) (end 114.078647 69.921353) (width 0.25) (layer "F.Cu") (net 5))
 (segment (start 79.3 66.96) (end 80.045 67.705) (width 0.25) (layer "F.Cu") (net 5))
 (segment (start 78.74 83.82) (end 81.84 86.92) (width 1) (layer "F.Cu") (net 1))
 (segment (start 78.74 81.28) (end 78.74 83.82) (width 1) (layer "F.Cu") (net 1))
 (segment (start 81.84 86.92) (end 89.46 86.92) (width 1) (layer "F.Cu") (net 1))
 (segment (start 114.86 43.74) (end 119.94 43.74) (width 0.25) (layer "F.Cu") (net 15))
 (segment (start 119.94 43.74) (end 129.54 53.34) (width 0.25) (layer "F.Cu") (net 15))
 (segment (start 129.54 53.34) (end 142.24 53.34) (width 0.25) (layer "F.Cu") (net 15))
 (segment (start 142.8 52.78) (end 142.8 48.26) (width 0.25) (layer "F.Cu") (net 15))
 (segment (start 142.24 53.34) (end 142.8 52.78) (width 0.25) (layer "F.Cu") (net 15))
 (segment (start 145.34 57.86) (end 145.34 48.26) (width 0.25) (layer "F.Cu") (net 14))
 (segment (start 114.86 58.98) (end 144.22 58.98) (width 0.25) (layer "F.Cu") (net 14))
 (segment (start 144.22 58.98) (end 145.34 57.86) (width 0.25) (layer "F.Cu") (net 14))
 (segment (start 144.22 61.52) (end 147.88 57.86) (width 0.25) (layer "F.Cu") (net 13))
 (segment (start 147.88 57.86) (end 147.88 48.26) (width 0.25) (layer "F.Cu") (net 13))
 (segment (start 114.86 61.52) (end 144.22 61.52) (width 0.25) (layer "F.Cu") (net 13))
 (segment (start 142.8 76.2) (end 127 76.2) (width 0.25) (layer "F.Cu") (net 6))
 (segment (start 127 76.2) (end 114.86 64.06) (width 0.25) (layer "F.Cu") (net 6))
 (segment (start 145.34 73.66) (end 142.8 76.2) (width 0.25) (layer "F.Cu") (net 6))
 (segment (start 104.14 78.74) (end 111.2 71.68) (width 0.25) (layer "F.Cu") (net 16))
 (segment (start 111.2 71.68) (end 114.86 71.68) (width 0.25) (layer "F.Cu") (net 16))
 (segment (start 140.26 45.16) (end 142.24 43.18) (width 0.25) (layer "F.Cu") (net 16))
 (segment (start 140.26 48.26) (end 140.26 45.16) (width 0.25) (layer "F.Cu") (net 16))
 (segment (start 142.24 43.18) (end 160.02 43.18) (width 0.25) (layer "F.Cu") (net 16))
 (segment (start 104.14 88.9) (end 104.14 78.74) (width 0.25) (layer "F.Cu") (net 16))
 (segment (start 109.22 93.98) (end 104.14 88.9) (width 0.25) (layer "F.Cu") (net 16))
 (segment (start 160.02 43.18) (end 162.56 45.72) (width 0.25) (layer "F.Cu") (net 16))
 (segment (start 144.78 93.98) (end 109.22 93.98) (width 0.25) (layer "F.Cu") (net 16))
 (segment (start 162.56 76.2) (end 144.78 93.98) (width 0.25) (layer "F.Cu") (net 16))
 (segment (start 162.56 45.72) (end 162.56 76.2) (width 0.25) (layer "F.Cu") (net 16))
 (segment (start 145.34 78.74) (end 147.88 76.2) (width 0.25) (layer "F.Cu") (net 7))
 (segment (start 116.84 78.74) (end 145.34 78.74) (width 0.25) (layer "F.Cu") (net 7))
 (segment (start 147.88 76.2) (end 147.88 73.66) (width 0.25) (layer "F.Cu") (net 7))
 (segment (start 114.86 76.76) (end 116.84 78.74) (width 0.25) (layer "F.Cu") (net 7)))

